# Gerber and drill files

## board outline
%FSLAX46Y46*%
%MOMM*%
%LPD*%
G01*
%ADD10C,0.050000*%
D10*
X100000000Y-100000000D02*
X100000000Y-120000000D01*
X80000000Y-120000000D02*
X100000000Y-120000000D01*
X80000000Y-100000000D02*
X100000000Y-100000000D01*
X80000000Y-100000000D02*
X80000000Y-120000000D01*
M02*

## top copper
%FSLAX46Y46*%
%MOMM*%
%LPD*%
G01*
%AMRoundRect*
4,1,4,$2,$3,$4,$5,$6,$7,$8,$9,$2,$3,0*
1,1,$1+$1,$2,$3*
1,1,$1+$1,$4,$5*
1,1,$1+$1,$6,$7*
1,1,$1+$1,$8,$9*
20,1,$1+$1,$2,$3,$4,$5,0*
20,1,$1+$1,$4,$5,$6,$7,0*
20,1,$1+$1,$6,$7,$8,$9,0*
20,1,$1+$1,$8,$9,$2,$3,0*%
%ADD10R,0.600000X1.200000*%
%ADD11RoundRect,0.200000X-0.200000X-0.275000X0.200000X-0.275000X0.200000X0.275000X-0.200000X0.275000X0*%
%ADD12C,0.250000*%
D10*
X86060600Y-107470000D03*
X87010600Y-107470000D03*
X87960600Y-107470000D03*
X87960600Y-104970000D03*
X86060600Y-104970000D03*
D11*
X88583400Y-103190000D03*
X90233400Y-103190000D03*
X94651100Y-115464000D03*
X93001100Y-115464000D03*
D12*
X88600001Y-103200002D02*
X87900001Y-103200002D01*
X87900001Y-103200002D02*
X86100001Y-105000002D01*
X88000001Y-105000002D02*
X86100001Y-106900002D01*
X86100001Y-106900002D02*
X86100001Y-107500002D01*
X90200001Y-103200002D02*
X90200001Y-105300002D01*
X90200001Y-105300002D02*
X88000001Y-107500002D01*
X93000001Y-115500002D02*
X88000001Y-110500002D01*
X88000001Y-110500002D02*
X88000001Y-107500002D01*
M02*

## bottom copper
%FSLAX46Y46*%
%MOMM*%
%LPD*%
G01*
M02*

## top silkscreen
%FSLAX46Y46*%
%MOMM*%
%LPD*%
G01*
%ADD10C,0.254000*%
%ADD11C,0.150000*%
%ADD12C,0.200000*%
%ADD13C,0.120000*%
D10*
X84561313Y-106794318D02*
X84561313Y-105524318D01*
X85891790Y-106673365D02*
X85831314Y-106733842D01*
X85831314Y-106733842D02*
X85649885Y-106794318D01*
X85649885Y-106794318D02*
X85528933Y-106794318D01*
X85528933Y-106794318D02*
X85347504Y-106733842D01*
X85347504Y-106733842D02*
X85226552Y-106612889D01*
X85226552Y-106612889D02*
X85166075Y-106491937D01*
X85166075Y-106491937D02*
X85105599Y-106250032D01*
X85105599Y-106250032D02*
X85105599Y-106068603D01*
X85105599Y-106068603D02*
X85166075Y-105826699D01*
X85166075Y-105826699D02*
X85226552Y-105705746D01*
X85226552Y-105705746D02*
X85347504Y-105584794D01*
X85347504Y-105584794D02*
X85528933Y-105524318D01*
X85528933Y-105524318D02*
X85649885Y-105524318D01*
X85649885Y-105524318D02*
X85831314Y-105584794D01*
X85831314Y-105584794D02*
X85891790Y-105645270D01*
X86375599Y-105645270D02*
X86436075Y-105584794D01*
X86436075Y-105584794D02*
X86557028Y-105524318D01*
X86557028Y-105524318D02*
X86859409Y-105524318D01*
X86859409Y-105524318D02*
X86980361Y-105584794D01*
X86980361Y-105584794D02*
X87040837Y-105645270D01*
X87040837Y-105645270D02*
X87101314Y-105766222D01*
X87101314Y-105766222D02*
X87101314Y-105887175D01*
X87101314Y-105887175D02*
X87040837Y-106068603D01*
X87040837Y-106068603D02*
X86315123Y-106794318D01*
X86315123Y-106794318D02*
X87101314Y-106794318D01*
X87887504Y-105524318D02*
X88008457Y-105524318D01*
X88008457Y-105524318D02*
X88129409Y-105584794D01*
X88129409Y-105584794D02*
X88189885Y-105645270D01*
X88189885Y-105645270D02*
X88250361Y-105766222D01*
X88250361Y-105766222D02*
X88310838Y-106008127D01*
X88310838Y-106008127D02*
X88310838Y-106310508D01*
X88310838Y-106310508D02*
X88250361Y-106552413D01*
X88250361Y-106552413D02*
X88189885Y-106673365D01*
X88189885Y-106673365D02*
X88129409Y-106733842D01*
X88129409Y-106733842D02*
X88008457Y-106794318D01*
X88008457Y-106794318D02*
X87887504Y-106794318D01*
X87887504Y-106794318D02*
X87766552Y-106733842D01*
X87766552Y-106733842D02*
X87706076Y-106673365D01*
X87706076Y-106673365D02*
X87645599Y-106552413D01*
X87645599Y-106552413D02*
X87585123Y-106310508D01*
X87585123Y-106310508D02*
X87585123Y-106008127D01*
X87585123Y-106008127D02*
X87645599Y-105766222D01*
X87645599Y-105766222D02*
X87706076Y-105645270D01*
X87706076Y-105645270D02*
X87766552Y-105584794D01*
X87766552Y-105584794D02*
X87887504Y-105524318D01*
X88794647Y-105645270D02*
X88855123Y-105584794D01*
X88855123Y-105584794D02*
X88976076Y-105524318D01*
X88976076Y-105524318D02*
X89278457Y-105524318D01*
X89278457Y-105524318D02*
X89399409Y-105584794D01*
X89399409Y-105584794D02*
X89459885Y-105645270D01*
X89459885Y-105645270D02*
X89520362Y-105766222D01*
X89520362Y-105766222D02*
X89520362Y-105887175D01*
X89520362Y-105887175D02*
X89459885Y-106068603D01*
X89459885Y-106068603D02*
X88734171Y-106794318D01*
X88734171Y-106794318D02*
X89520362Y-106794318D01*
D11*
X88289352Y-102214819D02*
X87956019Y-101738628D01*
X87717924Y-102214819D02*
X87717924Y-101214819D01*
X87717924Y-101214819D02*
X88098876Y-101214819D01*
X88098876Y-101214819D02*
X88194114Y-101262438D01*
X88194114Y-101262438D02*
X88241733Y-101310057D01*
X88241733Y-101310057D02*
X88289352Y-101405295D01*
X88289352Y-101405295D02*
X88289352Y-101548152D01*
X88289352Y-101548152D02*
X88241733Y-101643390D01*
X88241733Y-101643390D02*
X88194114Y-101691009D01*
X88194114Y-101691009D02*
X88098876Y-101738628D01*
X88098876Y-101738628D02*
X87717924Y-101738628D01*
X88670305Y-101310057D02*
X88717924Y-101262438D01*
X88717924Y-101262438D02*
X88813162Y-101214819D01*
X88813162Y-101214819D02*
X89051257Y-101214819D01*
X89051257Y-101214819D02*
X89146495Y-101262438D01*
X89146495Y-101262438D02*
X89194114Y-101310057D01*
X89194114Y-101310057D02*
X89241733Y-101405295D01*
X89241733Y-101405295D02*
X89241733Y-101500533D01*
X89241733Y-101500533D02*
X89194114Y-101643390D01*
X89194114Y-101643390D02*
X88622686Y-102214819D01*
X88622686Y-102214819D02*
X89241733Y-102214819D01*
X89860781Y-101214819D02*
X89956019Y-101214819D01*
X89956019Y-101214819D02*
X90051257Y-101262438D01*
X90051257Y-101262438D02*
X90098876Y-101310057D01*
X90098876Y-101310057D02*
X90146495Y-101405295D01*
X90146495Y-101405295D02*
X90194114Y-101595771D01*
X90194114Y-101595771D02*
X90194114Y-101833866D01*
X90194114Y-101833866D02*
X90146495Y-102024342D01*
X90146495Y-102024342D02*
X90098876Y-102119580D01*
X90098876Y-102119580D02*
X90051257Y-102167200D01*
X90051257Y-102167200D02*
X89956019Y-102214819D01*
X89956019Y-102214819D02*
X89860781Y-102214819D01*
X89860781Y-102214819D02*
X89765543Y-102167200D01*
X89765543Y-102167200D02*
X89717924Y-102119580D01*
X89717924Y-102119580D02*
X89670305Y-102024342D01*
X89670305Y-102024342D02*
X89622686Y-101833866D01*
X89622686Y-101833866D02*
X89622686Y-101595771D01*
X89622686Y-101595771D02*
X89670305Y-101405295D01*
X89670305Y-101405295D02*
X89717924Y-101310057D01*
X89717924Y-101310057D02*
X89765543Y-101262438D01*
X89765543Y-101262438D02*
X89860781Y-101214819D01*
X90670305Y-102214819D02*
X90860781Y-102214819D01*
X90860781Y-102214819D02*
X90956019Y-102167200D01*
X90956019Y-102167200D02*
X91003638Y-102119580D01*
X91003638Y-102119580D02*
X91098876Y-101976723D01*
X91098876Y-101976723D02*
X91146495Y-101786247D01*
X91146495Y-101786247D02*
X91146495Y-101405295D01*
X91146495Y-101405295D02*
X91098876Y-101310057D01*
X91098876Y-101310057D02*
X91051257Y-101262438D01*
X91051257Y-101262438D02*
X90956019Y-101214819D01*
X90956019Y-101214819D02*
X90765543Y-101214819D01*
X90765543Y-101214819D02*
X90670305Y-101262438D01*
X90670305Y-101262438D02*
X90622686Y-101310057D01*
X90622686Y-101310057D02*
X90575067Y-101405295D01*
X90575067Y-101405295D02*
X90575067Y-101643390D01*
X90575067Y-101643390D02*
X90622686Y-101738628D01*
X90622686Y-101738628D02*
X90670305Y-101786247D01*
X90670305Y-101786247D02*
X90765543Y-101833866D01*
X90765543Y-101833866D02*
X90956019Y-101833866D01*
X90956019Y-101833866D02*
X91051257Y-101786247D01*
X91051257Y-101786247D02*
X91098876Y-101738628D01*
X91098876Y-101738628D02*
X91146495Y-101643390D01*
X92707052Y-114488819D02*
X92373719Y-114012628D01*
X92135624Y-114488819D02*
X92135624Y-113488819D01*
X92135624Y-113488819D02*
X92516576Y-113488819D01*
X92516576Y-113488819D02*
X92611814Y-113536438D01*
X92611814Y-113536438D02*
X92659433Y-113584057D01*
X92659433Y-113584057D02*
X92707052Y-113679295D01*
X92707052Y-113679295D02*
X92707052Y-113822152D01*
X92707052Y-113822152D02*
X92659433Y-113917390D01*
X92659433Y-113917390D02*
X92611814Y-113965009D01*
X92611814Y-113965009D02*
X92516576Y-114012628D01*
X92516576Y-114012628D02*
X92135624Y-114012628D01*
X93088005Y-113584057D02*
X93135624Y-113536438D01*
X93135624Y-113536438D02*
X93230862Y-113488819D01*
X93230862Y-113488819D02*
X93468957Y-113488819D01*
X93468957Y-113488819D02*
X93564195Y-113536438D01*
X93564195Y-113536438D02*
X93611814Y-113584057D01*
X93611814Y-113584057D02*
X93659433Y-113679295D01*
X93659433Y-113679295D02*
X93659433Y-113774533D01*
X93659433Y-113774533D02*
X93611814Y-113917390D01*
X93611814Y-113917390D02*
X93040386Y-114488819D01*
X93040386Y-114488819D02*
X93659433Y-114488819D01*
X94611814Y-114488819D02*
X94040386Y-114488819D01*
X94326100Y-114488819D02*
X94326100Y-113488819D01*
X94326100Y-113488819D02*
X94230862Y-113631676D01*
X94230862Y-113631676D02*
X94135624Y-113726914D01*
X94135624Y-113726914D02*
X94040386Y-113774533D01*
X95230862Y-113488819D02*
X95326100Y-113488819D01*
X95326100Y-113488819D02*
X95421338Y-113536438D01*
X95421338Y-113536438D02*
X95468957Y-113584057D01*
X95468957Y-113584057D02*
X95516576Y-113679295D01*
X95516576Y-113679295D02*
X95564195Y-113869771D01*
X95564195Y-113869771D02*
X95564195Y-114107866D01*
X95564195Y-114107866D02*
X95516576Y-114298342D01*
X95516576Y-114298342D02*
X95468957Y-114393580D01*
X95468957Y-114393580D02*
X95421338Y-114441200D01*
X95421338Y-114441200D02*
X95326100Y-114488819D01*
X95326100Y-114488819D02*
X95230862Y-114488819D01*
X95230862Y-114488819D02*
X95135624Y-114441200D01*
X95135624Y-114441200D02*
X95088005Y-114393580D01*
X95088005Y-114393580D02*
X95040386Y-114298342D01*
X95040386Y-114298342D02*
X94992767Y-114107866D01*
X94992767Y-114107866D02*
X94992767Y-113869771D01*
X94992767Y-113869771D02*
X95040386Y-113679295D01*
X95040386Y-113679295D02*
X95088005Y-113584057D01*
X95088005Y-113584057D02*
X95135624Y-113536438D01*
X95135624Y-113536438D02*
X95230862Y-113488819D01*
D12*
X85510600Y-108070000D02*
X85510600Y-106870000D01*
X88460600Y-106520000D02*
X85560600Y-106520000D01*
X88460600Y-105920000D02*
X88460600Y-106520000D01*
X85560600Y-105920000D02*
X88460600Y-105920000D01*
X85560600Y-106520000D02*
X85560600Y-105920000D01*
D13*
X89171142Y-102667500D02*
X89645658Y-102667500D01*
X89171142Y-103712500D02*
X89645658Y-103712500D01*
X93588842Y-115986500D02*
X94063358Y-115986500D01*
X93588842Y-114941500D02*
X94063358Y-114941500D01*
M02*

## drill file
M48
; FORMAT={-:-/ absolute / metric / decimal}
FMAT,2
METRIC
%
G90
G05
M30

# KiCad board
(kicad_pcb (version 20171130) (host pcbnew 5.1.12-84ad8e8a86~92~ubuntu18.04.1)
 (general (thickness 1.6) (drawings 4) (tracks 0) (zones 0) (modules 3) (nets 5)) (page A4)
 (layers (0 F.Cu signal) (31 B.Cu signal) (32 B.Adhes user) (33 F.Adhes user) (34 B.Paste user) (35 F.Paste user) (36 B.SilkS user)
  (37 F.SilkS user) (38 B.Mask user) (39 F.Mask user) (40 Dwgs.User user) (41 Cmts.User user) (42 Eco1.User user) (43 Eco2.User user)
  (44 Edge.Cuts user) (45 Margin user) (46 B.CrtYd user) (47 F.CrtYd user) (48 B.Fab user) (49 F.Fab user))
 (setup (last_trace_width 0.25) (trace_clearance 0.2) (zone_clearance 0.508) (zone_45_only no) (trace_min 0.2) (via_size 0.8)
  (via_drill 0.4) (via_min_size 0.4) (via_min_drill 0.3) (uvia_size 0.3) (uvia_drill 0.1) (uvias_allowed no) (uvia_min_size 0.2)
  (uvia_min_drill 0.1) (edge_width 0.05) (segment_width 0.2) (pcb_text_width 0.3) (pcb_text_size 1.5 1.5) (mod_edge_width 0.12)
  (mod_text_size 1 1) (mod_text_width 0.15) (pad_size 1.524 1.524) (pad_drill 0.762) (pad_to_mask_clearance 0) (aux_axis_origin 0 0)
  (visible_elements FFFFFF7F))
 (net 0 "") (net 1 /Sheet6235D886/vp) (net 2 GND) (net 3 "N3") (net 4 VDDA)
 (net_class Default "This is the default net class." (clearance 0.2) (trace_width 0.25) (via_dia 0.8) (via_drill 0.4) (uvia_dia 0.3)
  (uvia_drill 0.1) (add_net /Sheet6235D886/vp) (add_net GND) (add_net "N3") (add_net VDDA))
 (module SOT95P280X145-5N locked (layer F.Cu) (at 87.010600 106.220000 90.000000)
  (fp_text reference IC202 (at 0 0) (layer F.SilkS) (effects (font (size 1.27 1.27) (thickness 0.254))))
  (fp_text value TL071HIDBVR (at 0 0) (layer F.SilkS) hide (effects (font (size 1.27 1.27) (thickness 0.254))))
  (fp_line (start -1.85 -1.5) (end -0.65 -1.5) (layer F.SilkS) (width 0.2))
  (fp_line (start -0.3 1.45) (end -0.3 -1.45) (layer F.SilkS) (width 0.2))
  (fp_line (start 0.3 1.45) (end -0.3 1.45) (layer F.SilkS) (width 0.2))
  (fp_line (start 0.3 -1.45) (end 0.3 1.45) (layer F.SilkS) (width 0.2))
  (fp_line (start -0.3 -1.45) (end 0.3 -1.45) (layer F.SilkS) (width 0.2))
  (pad 1 smd rect (at -1.25 -0.95 180.000000) (size 0.6 1.2) (layers F.Cu F.Mask F.Paste) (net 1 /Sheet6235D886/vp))
  (pad 2 smd rect (at -1.25 0 180.000000) (size 0.6 1.2) (layers F.Cu F.Mask F.Paste) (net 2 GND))
  (pad 3 smd rect (at -1.25 0.95 180.000000) (size 0.6 1.2) (layers F.Cu F.Mask F.Paste) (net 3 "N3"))
  (pad 4 smd rect (at 1.25 0.95 180.000000) (size 0.6 1.2) (layers F.Cu F.Mask F.Paste) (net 1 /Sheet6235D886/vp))
  (pad 5 smd rect (at 1.25 -0.95 180.000000) (size 0.6 1.2) (layers F.Cu F.Mask F.Paste) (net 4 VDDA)))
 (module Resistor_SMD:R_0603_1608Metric (layer F.Cu) (at 89.408400 103.190000)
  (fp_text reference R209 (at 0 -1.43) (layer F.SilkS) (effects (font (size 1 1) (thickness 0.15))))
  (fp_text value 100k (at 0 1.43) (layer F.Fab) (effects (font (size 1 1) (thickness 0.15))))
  (fp_line (start -0.237258 -0.5225) (end 0.237258 -0.5225) (layer F.SilkS) (width 0.12))
  (fp_line (start -0.237258 0.5225) (end 0.237258 0.5225) (layer F.SilkS) (width 0.12))
  (pad 1 smd roundrect (at -0.825 0) (size 0.8 0.95) (layers F.Cu F.Mask F.Paste) (roundrect_rratio 0.25) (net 4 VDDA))
  (pad 2 smd roundrect (at 0.825 0) (size 0.8 0.95) (layers F.Cu F.Mask F.Paste) (roundrect_rratio 0.25) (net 3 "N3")))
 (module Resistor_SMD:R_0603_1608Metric (layer F.Cu) (at 93.826100 115.464000)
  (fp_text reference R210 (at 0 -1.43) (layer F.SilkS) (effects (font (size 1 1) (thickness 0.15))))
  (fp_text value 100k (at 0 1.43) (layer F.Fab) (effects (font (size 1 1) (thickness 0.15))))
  (fp_line (start -0.237258 0.5225) (end 0.237258 0.5225) (layer F.SilkS) (width 0.12))
  (fp_line (start -0.237258 -0.5225) (end 0.237258 -0.5225) (layer F.SilkS) (width 0.12))
  (pad 2 smd roundrect (at 0.825 0) (size 0.8 0.95) (layers F.Cu F.Mask F.Paste) (roundrect_rratio 0.25) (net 2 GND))
  (pad 1 smd roundrect (at -0.825 0) (size 0.8 0.95) (layers F.Cu F.Mask F.Paste) (roundrect_rratio 0.25) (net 3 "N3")))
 (gr_line (start 100 100) (end 100 120) (layer Edge.Cuts) (width 0.05))
 (gr_line (start 80 120) (end 100 120) (layer Edge.Cuts) (width 0.05))
 (gr_line (start 80 100) (end 100 100) (layer Edge.Cuts) (width 0.05))
 (gr_line (start 80 100) (end 80 120) (layer Edge.Cuts) (width 0.05))
 (segment (start 88.600001 103.200002) (end 87.900001 103.200002) (width 0.250000) (layer F.Cu) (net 4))
 (segment (start 87.900001 103.200002) (end 86.100001 105.000002) (width 0.250000) (layer F.Cu) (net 4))
 (segment (start 88.000001 105.000002) (end 86.100001 106.900002) (width 0.250000) (layer F.Cu) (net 1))
 (segment (start 86.100001 106.900002) (end 86.100001 107.500002) (width 0.250000) (layer F.Cu) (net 1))
 (segment (start 90.200001 103.200002) (end 90.200001 105.300002) (width 0.250000) (layer F.Cu) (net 3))
 (segment (start 90.200001 105.300002) (end 88.000001 107.500002) (width 0.250000) (layer F.Cu) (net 3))
 (segment (start 93.000001 115.500002) (end 88.000001 110.500002) (width 0.250000) (layer F.Cu) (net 3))
 (segment (start 88.000001 110.500002) (end 88.000001 107.500002) (width 0.250000) (layer F.Cu) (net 3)))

